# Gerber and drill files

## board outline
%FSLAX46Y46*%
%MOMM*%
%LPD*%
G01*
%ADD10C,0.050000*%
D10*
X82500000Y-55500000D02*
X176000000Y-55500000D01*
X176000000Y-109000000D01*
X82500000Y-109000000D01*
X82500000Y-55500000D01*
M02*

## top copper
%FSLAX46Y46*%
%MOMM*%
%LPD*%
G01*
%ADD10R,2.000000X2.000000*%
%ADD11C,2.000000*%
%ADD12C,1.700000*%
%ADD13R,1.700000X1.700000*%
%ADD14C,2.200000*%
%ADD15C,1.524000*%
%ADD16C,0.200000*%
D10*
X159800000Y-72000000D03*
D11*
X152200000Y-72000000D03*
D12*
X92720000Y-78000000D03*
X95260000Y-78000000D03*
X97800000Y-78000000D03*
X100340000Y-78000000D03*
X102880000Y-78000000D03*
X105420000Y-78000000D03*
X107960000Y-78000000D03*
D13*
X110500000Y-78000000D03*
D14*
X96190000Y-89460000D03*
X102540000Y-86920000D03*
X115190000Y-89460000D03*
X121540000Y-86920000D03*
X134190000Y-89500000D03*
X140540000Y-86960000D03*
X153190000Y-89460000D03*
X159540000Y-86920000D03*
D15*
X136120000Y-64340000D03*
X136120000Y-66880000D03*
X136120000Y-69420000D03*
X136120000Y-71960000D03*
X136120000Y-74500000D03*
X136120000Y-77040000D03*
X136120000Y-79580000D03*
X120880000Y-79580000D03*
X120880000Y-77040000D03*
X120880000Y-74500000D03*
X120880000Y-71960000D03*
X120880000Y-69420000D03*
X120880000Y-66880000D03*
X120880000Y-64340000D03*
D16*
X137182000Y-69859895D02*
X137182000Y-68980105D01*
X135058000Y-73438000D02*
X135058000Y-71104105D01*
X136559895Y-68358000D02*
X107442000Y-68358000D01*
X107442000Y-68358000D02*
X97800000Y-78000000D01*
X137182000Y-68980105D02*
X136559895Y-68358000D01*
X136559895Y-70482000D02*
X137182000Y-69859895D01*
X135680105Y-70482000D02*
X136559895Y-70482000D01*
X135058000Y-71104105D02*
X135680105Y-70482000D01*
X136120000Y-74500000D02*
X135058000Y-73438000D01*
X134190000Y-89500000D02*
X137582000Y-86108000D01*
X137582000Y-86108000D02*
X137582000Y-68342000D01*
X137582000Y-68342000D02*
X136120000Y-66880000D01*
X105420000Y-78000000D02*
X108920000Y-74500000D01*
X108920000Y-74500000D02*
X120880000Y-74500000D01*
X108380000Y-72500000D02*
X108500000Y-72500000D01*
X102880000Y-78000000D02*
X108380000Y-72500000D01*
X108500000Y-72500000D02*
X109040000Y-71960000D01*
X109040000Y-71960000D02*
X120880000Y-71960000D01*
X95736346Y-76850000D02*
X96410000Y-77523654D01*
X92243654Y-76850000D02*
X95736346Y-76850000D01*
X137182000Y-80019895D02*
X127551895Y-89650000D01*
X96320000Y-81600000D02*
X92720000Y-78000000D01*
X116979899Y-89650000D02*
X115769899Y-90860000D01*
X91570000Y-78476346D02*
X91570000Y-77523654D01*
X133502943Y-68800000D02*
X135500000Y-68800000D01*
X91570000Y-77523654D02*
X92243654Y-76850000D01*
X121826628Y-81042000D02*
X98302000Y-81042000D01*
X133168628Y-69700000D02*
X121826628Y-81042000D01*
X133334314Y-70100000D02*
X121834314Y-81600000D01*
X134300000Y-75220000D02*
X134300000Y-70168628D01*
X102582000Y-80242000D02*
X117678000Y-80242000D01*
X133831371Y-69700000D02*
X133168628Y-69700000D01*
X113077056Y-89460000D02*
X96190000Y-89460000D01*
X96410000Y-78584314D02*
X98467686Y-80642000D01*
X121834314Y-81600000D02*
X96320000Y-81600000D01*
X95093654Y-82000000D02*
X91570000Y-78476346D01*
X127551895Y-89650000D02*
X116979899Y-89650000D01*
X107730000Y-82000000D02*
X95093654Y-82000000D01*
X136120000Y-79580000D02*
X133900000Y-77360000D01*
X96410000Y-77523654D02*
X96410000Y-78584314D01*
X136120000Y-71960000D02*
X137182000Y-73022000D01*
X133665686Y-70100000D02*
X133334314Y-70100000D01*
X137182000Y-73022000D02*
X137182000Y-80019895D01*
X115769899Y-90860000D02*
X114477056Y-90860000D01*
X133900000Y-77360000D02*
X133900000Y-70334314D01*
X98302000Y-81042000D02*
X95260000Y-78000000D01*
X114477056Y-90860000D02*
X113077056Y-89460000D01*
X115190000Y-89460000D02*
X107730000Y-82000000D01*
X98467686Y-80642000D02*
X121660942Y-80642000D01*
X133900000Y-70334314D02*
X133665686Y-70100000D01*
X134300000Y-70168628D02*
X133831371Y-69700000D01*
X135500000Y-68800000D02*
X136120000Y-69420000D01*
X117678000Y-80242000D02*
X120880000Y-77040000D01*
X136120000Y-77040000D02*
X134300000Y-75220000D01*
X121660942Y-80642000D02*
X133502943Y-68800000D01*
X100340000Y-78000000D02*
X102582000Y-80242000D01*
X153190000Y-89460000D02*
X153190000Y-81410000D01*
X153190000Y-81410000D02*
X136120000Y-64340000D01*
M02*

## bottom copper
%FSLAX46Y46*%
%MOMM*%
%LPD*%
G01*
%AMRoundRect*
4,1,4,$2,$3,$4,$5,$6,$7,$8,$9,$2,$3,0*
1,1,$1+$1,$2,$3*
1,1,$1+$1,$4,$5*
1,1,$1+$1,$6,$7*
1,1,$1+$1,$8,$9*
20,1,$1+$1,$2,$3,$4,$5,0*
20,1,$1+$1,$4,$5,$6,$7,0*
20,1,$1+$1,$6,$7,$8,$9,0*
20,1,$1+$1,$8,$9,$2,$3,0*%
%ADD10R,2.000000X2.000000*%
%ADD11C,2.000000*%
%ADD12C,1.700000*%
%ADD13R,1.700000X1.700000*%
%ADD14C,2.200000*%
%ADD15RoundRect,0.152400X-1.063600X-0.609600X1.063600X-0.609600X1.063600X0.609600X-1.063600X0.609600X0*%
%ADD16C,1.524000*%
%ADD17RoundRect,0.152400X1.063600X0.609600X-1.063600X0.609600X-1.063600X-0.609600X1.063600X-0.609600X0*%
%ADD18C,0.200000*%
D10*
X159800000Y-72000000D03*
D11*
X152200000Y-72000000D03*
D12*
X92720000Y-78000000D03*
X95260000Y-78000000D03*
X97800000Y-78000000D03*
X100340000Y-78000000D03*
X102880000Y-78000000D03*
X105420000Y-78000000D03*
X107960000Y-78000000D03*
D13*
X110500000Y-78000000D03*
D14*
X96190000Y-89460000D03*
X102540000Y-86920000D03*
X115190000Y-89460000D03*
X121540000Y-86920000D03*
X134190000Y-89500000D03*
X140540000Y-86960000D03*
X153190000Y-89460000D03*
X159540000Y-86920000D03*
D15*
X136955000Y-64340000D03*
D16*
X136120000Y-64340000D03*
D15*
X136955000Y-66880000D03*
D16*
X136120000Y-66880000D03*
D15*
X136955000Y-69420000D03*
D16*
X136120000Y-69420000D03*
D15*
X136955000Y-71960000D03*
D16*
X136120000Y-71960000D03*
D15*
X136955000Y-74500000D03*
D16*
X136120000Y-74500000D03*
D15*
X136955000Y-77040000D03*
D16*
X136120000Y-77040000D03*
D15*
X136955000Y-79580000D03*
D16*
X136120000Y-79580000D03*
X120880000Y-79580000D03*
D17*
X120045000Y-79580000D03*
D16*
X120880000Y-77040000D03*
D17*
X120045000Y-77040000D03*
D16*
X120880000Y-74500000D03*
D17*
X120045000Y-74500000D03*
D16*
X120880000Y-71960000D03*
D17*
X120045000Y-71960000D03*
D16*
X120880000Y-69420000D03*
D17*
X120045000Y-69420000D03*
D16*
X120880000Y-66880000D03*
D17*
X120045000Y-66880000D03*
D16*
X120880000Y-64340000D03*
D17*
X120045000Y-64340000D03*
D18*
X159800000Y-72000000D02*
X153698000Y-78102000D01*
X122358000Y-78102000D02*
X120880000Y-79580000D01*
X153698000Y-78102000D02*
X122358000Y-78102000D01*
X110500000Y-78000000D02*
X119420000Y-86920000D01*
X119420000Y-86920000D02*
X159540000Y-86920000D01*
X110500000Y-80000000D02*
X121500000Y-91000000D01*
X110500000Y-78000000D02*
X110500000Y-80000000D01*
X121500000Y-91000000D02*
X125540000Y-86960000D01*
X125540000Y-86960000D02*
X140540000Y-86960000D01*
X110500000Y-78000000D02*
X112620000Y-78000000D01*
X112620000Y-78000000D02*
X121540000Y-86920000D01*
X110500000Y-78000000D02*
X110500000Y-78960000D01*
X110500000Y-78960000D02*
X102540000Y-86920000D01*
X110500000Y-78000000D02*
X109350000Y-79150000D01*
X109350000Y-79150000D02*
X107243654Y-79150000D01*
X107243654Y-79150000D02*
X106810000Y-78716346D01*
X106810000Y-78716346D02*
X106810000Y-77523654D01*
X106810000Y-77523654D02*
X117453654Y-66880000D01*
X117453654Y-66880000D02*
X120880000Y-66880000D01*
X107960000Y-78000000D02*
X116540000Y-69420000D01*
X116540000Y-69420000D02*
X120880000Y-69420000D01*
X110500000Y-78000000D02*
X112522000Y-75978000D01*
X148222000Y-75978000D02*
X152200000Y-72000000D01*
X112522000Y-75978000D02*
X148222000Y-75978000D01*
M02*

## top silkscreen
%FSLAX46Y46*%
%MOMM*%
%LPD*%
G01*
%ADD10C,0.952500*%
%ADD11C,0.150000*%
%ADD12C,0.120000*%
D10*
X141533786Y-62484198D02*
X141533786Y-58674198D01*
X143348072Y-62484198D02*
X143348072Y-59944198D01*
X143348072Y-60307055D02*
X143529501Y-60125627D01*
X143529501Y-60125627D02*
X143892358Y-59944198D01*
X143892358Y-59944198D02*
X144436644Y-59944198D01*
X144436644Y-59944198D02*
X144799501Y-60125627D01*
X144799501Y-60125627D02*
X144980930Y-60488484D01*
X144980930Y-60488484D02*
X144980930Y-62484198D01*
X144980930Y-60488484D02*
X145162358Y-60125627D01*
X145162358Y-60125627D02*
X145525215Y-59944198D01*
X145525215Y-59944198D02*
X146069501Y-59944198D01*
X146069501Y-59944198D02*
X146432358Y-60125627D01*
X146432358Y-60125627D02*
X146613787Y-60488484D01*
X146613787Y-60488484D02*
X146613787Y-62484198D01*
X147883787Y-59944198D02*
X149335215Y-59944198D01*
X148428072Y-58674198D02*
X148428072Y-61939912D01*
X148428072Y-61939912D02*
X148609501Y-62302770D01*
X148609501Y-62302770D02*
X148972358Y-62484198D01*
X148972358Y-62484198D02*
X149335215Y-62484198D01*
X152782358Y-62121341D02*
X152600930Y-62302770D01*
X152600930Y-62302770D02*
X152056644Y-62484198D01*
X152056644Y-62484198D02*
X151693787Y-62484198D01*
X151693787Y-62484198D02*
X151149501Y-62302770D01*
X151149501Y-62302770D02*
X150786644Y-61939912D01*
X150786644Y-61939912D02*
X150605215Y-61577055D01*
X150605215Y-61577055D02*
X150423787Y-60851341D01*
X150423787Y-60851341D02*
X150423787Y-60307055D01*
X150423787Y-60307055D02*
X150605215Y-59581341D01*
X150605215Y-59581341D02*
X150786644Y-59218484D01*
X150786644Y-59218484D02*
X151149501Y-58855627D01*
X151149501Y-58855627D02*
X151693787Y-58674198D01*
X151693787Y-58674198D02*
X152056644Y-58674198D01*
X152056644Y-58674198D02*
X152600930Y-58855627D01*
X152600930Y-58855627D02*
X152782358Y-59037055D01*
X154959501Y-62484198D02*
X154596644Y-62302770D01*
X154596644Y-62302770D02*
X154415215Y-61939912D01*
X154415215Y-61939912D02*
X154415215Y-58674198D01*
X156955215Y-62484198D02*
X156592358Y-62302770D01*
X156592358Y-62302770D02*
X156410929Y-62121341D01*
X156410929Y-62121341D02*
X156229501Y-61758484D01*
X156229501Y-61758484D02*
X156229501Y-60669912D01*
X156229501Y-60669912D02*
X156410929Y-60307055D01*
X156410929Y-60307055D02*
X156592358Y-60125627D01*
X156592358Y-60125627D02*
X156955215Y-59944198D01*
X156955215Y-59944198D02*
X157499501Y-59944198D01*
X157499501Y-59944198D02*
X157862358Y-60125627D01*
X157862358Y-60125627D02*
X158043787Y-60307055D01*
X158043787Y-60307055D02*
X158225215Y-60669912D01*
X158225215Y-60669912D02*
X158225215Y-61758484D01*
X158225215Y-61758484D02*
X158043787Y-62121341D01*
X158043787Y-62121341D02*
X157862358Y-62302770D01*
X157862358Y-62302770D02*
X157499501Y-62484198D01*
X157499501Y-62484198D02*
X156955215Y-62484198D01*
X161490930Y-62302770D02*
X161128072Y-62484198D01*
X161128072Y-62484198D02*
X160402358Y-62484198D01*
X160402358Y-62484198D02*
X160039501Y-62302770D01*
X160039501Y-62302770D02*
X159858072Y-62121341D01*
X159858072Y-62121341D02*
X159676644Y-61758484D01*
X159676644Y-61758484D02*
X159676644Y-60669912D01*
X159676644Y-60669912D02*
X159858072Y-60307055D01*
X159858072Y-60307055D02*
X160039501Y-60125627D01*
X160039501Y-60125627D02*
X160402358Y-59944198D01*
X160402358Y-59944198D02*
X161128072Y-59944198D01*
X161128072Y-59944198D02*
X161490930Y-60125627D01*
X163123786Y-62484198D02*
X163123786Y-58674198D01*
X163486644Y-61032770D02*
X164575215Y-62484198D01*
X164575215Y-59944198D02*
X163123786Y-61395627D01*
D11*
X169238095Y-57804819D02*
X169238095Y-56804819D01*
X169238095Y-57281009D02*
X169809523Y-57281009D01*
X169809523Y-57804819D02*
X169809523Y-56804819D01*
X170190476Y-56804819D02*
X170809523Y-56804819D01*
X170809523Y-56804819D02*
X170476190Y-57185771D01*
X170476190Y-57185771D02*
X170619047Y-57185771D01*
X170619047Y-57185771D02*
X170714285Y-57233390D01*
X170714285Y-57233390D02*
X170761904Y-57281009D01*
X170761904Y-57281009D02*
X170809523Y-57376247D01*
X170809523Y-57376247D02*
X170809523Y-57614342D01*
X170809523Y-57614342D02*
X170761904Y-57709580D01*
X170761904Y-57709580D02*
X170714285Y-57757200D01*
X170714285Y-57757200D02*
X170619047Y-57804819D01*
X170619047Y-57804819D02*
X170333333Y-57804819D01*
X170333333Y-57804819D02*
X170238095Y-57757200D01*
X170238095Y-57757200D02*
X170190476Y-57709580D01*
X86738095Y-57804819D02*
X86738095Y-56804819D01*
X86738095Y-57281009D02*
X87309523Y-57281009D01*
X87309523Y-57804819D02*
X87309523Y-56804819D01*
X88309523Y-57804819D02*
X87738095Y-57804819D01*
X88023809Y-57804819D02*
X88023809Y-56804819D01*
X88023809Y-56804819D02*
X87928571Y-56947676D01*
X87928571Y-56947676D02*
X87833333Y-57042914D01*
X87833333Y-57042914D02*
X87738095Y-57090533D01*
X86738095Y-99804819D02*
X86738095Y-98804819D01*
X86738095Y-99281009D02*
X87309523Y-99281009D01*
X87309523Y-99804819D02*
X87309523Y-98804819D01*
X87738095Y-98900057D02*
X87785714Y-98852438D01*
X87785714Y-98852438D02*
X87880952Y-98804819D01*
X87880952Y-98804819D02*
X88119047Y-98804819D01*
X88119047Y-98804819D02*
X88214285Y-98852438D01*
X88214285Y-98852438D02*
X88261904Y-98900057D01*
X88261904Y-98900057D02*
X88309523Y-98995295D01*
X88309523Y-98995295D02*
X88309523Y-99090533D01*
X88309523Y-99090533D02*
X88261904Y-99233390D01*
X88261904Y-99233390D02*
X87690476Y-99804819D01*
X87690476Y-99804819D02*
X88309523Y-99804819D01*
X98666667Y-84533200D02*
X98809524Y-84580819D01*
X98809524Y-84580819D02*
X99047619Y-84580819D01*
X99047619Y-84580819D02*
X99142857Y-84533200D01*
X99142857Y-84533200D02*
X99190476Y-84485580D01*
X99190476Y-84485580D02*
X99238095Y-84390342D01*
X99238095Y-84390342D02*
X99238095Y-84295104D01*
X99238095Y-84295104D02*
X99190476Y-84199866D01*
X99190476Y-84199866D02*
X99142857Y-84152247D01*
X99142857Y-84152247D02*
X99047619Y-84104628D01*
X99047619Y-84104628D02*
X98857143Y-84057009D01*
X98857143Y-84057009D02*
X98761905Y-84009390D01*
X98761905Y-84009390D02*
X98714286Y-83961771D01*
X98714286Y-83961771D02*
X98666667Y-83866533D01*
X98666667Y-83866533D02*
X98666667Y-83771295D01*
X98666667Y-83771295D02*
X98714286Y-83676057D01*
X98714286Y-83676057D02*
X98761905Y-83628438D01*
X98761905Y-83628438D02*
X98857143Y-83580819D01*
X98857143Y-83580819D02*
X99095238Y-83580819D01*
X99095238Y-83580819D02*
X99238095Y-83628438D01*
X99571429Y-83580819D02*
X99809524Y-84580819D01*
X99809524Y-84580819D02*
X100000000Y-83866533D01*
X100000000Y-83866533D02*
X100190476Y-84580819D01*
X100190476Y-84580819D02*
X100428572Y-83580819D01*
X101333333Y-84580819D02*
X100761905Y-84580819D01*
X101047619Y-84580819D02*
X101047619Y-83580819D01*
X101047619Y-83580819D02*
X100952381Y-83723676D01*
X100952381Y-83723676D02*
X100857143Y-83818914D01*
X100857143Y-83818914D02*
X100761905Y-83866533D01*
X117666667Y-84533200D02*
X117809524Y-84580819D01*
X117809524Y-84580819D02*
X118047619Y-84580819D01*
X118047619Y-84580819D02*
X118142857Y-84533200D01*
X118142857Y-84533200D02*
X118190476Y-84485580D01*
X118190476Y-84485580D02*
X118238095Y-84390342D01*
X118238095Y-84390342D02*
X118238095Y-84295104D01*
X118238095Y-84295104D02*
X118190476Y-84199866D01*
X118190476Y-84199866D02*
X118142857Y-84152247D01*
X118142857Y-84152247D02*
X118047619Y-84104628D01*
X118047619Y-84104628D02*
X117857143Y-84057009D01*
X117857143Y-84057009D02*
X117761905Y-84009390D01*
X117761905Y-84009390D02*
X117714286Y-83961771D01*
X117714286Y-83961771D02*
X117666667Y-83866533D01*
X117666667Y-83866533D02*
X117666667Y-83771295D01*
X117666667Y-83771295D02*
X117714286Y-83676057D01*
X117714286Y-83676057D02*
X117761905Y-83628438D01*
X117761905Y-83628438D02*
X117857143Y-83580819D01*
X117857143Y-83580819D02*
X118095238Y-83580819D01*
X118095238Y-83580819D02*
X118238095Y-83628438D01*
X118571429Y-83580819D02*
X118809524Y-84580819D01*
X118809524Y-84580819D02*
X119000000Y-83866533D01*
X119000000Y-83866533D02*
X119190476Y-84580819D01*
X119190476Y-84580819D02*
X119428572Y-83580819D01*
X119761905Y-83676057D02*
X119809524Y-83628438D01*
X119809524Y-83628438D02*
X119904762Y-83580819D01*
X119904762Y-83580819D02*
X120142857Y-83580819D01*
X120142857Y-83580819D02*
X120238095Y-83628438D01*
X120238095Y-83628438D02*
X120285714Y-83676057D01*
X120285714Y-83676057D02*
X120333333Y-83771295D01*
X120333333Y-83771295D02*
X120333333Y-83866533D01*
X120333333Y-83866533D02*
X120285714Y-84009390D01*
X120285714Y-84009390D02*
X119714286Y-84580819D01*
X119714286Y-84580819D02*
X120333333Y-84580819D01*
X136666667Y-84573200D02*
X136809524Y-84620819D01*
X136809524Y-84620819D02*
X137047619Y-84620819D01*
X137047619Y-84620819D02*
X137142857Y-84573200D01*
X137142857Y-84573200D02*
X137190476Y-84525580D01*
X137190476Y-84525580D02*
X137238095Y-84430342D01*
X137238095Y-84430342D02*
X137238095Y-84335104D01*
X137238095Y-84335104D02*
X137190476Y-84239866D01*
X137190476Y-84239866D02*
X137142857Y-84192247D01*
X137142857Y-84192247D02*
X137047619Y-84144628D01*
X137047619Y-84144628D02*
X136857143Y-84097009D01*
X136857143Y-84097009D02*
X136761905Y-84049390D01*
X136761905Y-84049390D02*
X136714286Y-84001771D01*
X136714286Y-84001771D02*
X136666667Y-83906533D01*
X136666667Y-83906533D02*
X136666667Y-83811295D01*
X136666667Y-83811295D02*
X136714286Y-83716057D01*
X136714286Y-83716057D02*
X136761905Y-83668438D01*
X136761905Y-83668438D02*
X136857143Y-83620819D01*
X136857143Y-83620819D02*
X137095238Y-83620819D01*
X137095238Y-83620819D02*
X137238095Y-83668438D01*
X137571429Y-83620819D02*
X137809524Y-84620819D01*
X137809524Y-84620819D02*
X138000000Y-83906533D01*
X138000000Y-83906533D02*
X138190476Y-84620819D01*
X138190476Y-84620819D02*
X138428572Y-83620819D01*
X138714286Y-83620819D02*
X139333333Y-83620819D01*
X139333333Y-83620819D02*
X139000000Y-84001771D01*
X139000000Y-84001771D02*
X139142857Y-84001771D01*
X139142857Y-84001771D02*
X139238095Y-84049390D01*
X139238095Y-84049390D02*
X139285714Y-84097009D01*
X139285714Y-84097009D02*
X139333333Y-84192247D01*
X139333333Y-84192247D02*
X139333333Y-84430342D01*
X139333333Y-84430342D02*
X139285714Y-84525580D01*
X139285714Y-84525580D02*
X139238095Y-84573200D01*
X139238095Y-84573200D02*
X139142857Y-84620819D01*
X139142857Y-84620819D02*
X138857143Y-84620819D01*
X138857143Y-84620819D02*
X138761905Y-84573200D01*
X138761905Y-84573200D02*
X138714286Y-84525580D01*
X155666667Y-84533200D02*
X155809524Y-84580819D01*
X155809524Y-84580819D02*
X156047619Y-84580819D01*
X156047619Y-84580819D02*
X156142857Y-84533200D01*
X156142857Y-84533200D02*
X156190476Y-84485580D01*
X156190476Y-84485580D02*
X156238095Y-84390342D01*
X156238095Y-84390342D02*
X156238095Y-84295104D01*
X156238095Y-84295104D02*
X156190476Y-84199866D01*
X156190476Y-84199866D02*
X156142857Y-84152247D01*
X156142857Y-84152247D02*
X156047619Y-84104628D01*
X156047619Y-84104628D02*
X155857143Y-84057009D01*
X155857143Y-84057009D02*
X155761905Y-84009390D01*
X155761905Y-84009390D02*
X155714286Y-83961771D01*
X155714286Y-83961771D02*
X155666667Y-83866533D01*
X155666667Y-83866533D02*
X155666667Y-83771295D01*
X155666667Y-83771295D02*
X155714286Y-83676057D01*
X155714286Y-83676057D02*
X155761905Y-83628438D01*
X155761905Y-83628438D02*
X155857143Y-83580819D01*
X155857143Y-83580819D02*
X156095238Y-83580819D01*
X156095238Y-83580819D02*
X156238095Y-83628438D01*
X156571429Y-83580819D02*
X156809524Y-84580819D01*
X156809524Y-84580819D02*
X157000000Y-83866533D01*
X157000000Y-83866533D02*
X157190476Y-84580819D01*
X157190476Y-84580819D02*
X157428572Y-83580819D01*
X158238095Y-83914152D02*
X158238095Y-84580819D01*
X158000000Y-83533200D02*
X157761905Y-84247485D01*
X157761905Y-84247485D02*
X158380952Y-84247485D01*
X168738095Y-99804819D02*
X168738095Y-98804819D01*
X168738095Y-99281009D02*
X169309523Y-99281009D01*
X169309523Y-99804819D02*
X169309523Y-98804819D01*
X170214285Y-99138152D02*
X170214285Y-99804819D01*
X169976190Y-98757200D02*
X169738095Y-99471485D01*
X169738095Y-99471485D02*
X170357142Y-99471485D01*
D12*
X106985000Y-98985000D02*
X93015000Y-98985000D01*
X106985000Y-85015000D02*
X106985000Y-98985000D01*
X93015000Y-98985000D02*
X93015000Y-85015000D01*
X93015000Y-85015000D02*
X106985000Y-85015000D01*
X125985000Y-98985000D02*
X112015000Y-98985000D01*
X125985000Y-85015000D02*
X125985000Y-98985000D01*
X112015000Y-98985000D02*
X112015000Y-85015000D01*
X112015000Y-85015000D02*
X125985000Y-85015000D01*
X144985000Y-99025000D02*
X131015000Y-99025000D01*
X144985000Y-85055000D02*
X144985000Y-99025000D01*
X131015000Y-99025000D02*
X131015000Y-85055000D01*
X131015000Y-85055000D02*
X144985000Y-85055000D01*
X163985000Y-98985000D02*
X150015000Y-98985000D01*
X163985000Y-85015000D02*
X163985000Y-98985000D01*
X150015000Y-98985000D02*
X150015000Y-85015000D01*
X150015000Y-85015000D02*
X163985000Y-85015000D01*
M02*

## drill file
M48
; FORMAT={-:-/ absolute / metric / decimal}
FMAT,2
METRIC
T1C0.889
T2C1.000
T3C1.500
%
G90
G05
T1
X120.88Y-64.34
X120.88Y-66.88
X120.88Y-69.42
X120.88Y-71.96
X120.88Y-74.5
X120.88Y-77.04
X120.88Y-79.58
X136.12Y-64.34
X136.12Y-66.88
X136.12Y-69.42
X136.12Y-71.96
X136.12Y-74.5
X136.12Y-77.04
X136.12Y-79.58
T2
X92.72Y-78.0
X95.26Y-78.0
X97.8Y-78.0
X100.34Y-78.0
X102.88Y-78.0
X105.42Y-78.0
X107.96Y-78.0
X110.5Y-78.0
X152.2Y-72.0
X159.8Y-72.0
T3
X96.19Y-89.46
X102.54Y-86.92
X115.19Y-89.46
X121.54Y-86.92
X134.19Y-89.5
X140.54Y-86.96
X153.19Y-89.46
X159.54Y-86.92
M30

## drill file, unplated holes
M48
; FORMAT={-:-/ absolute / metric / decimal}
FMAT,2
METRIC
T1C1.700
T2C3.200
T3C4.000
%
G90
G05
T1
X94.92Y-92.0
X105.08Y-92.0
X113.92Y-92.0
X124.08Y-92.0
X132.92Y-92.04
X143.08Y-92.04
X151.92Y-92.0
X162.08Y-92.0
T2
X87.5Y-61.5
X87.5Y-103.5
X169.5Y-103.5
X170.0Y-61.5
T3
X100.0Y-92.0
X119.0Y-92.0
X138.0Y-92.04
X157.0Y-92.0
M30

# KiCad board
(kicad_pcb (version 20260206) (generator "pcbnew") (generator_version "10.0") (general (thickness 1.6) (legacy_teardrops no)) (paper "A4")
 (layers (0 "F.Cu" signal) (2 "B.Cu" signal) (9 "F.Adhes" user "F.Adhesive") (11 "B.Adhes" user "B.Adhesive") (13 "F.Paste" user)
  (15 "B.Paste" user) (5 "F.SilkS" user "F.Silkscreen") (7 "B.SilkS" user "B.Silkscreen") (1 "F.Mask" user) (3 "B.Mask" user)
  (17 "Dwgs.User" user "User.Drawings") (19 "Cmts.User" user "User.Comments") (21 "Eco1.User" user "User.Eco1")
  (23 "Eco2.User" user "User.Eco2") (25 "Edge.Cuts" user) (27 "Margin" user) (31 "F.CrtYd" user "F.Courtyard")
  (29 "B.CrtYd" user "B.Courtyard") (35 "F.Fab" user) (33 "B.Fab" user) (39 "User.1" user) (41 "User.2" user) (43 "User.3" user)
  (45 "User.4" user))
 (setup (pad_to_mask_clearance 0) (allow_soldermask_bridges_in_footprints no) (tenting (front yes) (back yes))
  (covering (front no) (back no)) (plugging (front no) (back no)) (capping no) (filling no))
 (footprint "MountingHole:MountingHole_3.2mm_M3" (layer "F.Cu") (at 169.5 103.5)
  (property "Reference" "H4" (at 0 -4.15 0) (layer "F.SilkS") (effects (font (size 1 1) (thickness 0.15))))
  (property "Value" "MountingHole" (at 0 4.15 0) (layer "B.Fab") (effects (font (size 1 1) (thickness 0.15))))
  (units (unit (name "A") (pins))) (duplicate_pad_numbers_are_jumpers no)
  (pad "" np_thru_hole circle (at 0 0) (size 3.2 3.2) (drill 3.2) (layers "*.Cu" "*.Mask")))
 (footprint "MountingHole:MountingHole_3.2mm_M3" (layer "F.Cu") (at 87.5 61.5)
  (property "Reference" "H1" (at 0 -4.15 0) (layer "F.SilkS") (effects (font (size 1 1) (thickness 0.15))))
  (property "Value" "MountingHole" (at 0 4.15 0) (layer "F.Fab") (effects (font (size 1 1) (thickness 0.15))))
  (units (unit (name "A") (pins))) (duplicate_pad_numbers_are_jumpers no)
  (pad "" np_thru_hole circle (at 0 0) (size 3.2 3.2) (drill 3.2) (layers "*.Cu" "*.Mask")))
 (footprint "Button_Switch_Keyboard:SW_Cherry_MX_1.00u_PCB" (layer "F.Cu") (at 159.54 86.92)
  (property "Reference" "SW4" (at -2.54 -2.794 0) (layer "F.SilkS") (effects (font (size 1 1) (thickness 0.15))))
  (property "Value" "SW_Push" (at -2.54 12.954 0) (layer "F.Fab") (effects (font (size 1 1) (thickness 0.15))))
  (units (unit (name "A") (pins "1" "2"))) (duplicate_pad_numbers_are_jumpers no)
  (fp_line (start -9.525 -1.905) (end 4.445 -1.905) (stroke (width 0.12) (type solid)) (layer "F.SilkS"))
  (fp_line (start -9.525 12.065) (end -9.525 -1.905) (stroke (width 0.12) (type solid)) (layer "F.SilkS"))
  (fp_line (start 4.445 -1.905) (end 4.445 12.065) (stroke (width 0.12) (type solid)) (layer "F.SilkS"))
  (fp_line (start 4.445 12.065) (end -9.525 12.065) (stroke (width 0.12) (type solid)) (layer "F.SilkS"))
  (pad "" np_thru_hole circle (at -7.62 5.08) (size 1.7 1.7) (drill 1.7) (layers "*.Cu" "*.Mask"))
  (pad "" np_thru_hole circle (at -2.54 5.08) (size 4 4) (drill 4) (layers "*.Cu" "*.Mask"))
  (pad "" np_thru_hole circle (at 2.54 5.08) (size 1.7 1.7) (drill 1.7) (layers "*.Cu" "*.Mask"))
  (pad "1" thru_hole circle (at 0 0) (size 2.2 2.2) (drill 1.5) (layers "*.Cu" "*.Mask") (remove_unused_layers no) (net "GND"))
  (pad "2" thru_hole circle (at -6.35 2.54) (size 2.2 2.2) (drill 1.5) (layers "*.Cu" "*.Mask") (remove_unused_layers no)
   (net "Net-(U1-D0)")))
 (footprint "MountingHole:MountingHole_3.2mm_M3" (layer "F.Cu") (at 170 61.5)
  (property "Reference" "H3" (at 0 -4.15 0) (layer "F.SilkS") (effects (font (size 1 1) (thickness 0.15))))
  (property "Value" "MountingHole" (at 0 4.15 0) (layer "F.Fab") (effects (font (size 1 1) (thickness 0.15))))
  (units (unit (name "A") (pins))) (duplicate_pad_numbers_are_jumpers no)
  (pad "" np_thru_hole circle (at 0 0) (size 3.2 3.2) (drill 3.2) (layers "*.Cu" "*.Mask")))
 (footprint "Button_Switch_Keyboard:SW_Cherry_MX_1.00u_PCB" (layer "F.Cu") (at 140.54 86.96)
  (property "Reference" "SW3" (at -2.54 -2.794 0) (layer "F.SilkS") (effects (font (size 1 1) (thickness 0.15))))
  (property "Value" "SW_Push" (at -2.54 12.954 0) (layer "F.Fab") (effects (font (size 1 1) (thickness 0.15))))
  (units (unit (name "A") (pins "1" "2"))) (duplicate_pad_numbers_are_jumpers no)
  (fp_line (start -9.525 -1.905) (end 4.445 -1.905) (stroke (width 0.12) (type solid)) (layer "F.SilkS"))
  (fp_line (start -9.525 12.065) (end -9.525 -1.905) (stroke (width 0.12) (type solid)) (layer "F.SilkS"))
  (fp_line (start 4.445 -1.905) (end 4.445 12.065) (stroke (width 0.12) (type solid)) (layer "F.SilkS"))
  (fp_line (start 4.445 12.065) (end -9.525 12.065) (stroke (width 0.12) (type solid)) (layer "F.SilkS"))
  (pad "" np_thru_hole circle (at -7.62 5.08) (size 1.7 1.7) (drill 1.7) (layers "*.Cu" "*.Mask"))
  (pad "" np_thru_hole circle (at -2.54 5.08) (size 4 4) (drill 4) (layers "*.Cu" "*.Mask"))
  (pad "" np_thru_hole circle (at 2.54 5.08) (size 1.7 1.7) (drill 1.7) (layers "*.Cu" "*.Mask"))
  (pad "1" thru_hole circle (at 0 0) (size 2.2 2.2) (drill 1.5) (layers "*.Cu" "*.Mask") (remove_unused_layers no) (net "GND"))
  (pad "2" thru_hole circle (at -6.35 2.54) (size 2.2 2.2) (drill 1.5) (layers "*.Cu" "*.Mask") (remove_unused_layers no)
   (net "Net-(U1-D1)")))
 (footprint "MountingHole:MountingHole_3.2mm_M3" (layer "F.Cu") (at 87.5 103.5)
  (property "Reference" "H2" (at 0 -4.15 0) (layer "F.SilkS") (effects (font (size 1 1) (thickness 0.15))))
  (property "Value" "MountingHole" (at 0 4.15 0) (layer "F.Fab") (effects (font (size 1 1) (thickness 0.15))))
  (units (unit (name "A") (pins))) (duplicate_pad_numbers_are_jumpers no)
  (pad "" np_thru_hole circle (at 0 0) (size 3.2 3.2) (drill 3.2) (layers "*.Cu" "*.Mask")))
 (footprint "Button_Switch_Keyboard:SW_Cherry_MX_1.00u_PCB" (layer "F.Cu") (at 121.54 86.92)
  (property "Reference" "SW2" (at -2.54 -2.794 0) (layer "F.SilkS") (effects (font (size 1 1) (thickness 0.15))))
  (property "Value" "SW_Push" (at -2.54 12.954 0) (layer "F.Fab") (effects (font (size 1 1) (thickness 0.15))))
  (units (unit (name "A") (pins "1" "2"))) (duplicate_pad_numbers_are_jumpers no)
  (fp_line (start -9.525 -1.905) (end 4.445 -1.905) (stroke (width 0.12) (type solid)) (layer "F.SilkS"))
  (fp_line (start -9.525 12.065) (end -9.525 -1.905) (stroke (width 0.12) (type solid)) (layer "F.SilkS"))
  (fp_line (start 4.445 -1.905) (end 4.445 12.065) (stroke (width 0.12) (type solid)) (layer "F.SilkS"))
  (fp_line (start 4.445 12.065) (end -9.525 12.065) (stroke (width 0.12) (type solid)) (layer "F.SilkS"))
  (pad "" np_thru_hole circle (at -7.62 5.08) (size 1.7 1.7) (drill 1.7) (layers "*.Cu" "*.Mask"))
  (pad "" np_thru_hole circle (at -2.54 5.08) (size 4 4) (drill 4) (layers "*.Cu" "*.Mask"))
  (pad "" np_thru_hole circle (at 2.54 5.08) (size 1.7 1.7) (drill 1.7) (layers "*.Cu" "*.Mask"))
  (pad "1" thru_hole circle (at 0 0) (size 2.2 2.2) (drill 1.5) (layers "*.Cu" "*.Mask") (remove_unused_layers no) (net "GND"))
  (pad "2" thru_hole circle (at -6.35 2.54) (size 2.2 2.2) (drill 1.5) (layers "*.Cu" "*.Mask") (remove_unused_layers no)
   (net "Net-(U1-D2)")))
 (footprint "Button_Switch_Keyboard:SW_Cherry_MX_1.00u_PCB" (layer "F.Cu") (at 102.54 86.92)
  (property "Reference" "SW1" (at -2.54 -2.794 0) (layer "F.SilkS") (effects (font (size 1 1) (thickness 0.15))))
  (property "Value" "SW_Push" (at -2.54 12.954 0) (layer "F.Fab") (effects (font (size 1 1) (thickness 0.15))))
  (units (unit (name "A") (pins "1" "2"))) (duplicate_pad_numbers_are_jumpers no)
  (fp_line (start -9.525 -1.905) (end 4.445 -1.905) (stroke (width 0.12) (type solid)) (layer "F.SilkS"))
  (fp_line (start -9.525 12.065) (end -9.525 -1.905) (stroke (width 0.12) (type solid)) (layer "F.SilkS"))
  (fp_line (start 4.445 -1.905) (end 4.445 12.065) (stroke (width 0.12) (type solid)) (layer "F.SilkS"))
  (fp_line (start 4.445 12.065) (end -9.525 12.065) (stroke (width 0.12) (type solid)) (layer "F.SilkS"))
  (pad "" np_thru_hole circle (at -7.62 5.08) (size 1.7 1.7) (drill 1.7) (layers "*.Cu" "*.Mask"))
  (pad "" np_thru_hole circle (at -2.54 5.08) (size 4 4) (drill 4) (layers "*.Cu" "*.Mask"))
  (pad "" np_thru_hole circle (at 2.54 5.08) (size 1.7 1.7) (drill 1.7) (layers "*.Cu" "*.Mask"))
  (pad "1" thru_hole circle (at 0 0) (size 2.2 2.2) (drill 1.5) (layers "*.Cu" "*.Mask") (remove_unused_layers no) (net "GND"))
  (pad "2" thru_hole circle (at -6.35 2.54) (size 2.2 2.2) (drill 1.5) (layers "*.Cu" "*.Mask") (remove_unused_layers no)
   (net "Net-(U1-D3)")))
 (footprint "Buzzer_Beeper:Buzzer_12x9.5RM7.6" (layer "B.Cu") (at 159.8 72 180)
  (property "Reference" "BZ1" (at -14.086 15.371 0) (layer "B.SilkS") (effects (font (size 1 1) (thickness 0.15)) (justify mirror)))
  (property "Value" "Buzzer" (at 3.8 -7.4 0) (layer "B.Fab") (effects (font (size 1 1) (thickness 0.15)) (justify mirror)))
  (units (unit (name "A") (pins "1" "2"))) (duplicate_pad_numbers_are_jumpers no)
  (pad "1" thru_hole rect (at 0 0 180) (size 2 2) (drill 1) (layers "*.Cu" "*.Mask") (remove_unused_layers no) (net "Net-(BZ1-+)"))
  (pad "2" thru_hole circle (at 7.6 0 180) (size 2 2) (drill 1) (layers "*.Cu" "*.Mask") (remove_unused_layers no) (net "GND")))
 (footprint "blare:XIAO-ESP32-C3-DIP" (layer "B.Cu") (at 128.5 71.96 90)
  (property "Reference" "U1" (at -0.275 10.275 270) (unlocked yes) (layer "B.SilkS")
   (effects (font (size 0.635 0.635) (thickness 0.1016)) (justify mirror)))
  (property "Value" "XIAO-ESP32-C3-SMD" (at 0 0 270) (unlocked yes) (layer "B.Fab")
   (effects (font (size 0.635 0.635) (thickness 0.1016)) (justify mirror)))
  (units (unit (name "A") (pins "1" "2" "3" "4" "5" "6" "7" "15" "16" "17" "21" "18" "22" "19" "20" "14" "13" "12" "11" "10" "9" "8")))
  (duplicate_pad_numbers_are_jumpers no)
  (pad "1" thru_hole circle (at 7.62 7.62) (size 1.524 1.524) (drill 0.889) (layers "*.Cu" "*.Mask") (remove_unused_layers no)
   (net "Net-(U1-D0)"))
  (pad "1" smd roundrect (at 7.62 8.455) (size 2.432 1.524) (layers "B.Cu" "B.Mask") (roundrect_rratio 0.1) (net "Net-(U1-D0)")
   (thermal_bridge_angle 45))
  (pad "2" thru_hole circle (at 5.08 7.62) (size 1.524 1.524) (drill 0.889) (layers "*.Cu" "*.Mask") (remove_unused_layers no)
   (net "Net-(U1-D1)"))
  (pad "2" smd roundrect (at 5.08 8.455) (size 2.432 1.524) (layers "B.Cu" "B.Mask") (roundrect_rratio 0.1) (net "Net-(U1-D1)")
   (thermal_bridge_angle 45))
  (pad "3" thru_hole circle (at 2.54 7.62) (size 1.524 1.524) (drill 0.889) (layers "*.Cu" "*.Mask") (remove_unused_layers no)
   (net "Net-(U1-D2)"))
  (pad "3" smd roundrect (at 2.54 8.455) (size 2.432 1.524) (layers "B.Cu" "B.Mask") (roundrect_rratio 0.1) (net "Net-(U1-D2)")
   (thermal_bridge_angle 45))
  (pad "4" thru_hole circle (at 0 7.62) (size 1.524 1.524) (drill 0.889) (layers "*.Cu" "*.Mask") (remove_unused_layers no)
   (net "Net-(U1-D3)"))
  (pad "4" smd roundrect (at 0 8.455) (size 2.432 1.524) (layers "B.Cu" "B.Mask") (roundrect_rratio 0.1) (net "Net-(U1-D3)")
   (thermal_bridge_angle 45))
  (pad "5" thru_hole circle (at -2.54 7.62) (size 1.524 1.524) (drill 0.889) (layers "*.Cu" "*.Mask") (remove_unused_layers no) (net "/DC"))
  (pad "5" smd roundrect (at -2.54 8.455) (size 2.432 1.524) (layers "B.Cu" "B.Mask") (roundrect_rratio 0.1) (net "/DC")
   (thermal_bridge_angle 45))
  (pad "6" thru_hole circle (at -5.08 7.62) (size 1.524 1.524) (drill 0.889) (layers "*.Cu" "*.Mask") (remove_unused_layers no) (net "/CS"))
  (pad "6" smd roundrect (at -5.08 8.455) (size 2.432 1.524) (layers "B.Cu" "B.Mask") (roundrect_rratio 0.1) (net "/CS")
   (thermal_bridge_angle 45))
  (pad "7" thru_hole circle (at -7.62 7.62) (size 1.524 1.524) (drill 0.889) (layers "*.Cu" "*.Mask") (remove_unused_layers no) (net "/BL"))
  (pad "7" smd roundrect (at -7.62 8.455) (size 2.432 1.524) (layers "B.Cu" "B.Mask") (roundrect_rratio 0.1) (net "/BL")
   (thermal_bridge_angle 45))
  (pad "8" smd roundrect (at -7.62 -8.455 180) (size 2.432 1.524) (layers "B.Cu" "B.Mask") (roundrect_rratio 0.1) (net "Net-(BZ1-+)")
   (thermal_bridge_angle 45))
  (pad "8" thru_hole circle (at -7.62 -7.62 180) (size 1.524 1.524) (drill 0.889) (layers "*.Cu" "*.Mask") (remove_unused_layers no)
   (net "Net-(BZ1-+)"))
  (pad "9" smd roundrect (at -5.08 -8.455 180) (size 2.432 1.524) (layers "B.Cu" "B.Mask") (roundrect_rratio 0.1) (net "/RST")
   (thermal_bridge_angle 45))
  (pad "9" thru_hole circle (at -5.08 -7.62 180) (size 1.524 1.524) (drill 0.889) (layers "*.Cu" "*.Mask") (remove_unused_layers no)
   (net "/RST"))
  (pad "10" smd roundrect (at -2.54 -8.455 180) (size 2.432 1.524) (layers "B.Cu" "B.Mask") (roundrect_rratio 0.1) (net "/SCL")
   (thermal_bridge_angle 45))
  (pad "10" thru_hole circle (at -2.54 -7.62 180) (size 1.524 1.524) (drill 0.889) (layers "*.Cu" "*.Mask") (remove_unused_layers no)
   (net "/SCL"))
  (pad "11" smd roundrect (at 0 -8.455 180) (size 2.432 1.524) (layers "B.Cu" "B.Mask") (roundrect_rratio 0.1) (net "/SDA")
   (thermal_bridge_angle 45))
  (pad "11" thru_hole circle (at 0 -7.62 180) (size 1.524 1.524) (drill 0.889) (layers "*.Cu" "*.Mask") (remove_unused_layers no)
   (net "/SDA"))
  (pad "12" smd roundrect (at 2.54 -8.455 180) (size 2.432 1.524) (layers "B.Cu" "B.Mask") (roundrect_rratio 0.1) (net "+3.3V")
   (thermal_bridge_angle 45))
  (pad "12" thru_hole circle (at 2.54 -7.62 180) (size 1.524 1.524) (drill 0.889) (layers "*.Cu" "*.Mask") (remove_unused_layers no)
   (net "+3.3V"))
  (pad "13" smd roundrect (at 5.08 -8.455 180) (size 2.432 1.524) (layers "B.Cu" "B.Mask") (roundrect_rratio 0.1) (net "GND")
   (thermal_bridge_angle 45))
  (pad "13" thru_hole circle (at 5.08 -7.62 180) (size 1.524 1.524) (drill 0.889) (layers "*.Cu" "*.Mask") (remove_unused_layers no)
   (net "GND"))
  (pad "14" smd roundrect (at 7.62 -8.455 180) (size 2.432 1.524) (layers "B.Cu" "B.Mask") (roundrect_rratio 0.1)
   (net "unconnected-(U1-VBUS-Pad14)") (thermal_bridge_angle 45))
  (pad "14" thru_hole circle (at 7.62 -7.62 180) (size 1.524 1.524) (drill 0.889) (layers "*.Cu" "*.Mask") (remove_unused_layers no)
   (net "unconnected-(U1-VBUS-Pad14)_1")))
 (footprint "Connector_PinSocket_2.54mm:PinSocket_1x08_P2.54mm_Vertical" (layer "B.Cu") (at 110.5 78 90)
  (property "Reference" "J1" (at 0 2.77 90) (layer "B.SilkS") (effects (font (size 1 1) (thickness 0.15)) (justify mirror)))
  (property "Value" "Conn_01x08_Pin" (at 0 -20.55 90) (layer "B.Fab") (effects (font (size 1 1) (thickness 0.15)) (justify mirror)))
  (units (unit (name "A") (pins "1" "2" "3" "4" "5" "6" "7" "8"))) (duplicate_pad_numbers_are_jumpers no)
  (pad "1" thru_hole rect (at 0 0 90) (size 1.7 1.7) (drill 1) (layers "*.Cu" "*.Mask") (remove_unused_layers no) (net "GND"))
  (pad "2" thru_hole circle (at 0 -2.54 90) (size 1.7 1.7) (drill 1) (layers "*.Cu" "*.Mask") (remove_unused_layers no) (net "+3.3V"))
  (pad "3" thru_hole circle (at 0 -5.08 90) (size 1.7 1.7) (drill 1) (layers "*.Cu" "*.Mask") (remove_unused_layers no) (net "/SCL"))
  (pad "4" thru_hole circle (at 0 -7.62 90) (size 1.7 1.7) (drill 1) (layers "*.Cu" "*.Mask") (remove_unused_layers no) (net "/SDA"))
  (pad "5" thru_hole circle (at 0 -10.16 90) (size 1.7 1.7) (drill 1) (layers "*.Cu" "*.Mask") (remove_unused_layers no) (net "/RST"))
  (pad "6" thru_hole circle (at 0 -12.7 90) (size 1.7 1.7) (drill 1) (layers "*.Cu" "*.Mask") (remove_unused_layers no) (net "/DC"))
  (pad "7" thru_hole circle (at 0 -15.24 90) (size 1.7 1.7) (drill 1) (layers "*.Cu" "*.Mask") (remove_unused_layers no) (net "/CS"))
  (pad "8" thru_hole circle (at 0 -17.78 90) (size 1.7 1.7) (drill 1) (layers "*.Cu" "*.Mask") (remove_unused_layers no) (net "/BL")))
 (gr_rect (start 82.5 55.5) (end 176 109) (stroke (width 0.05) (type default)) (fill no) (layer "Edge.Cuts"))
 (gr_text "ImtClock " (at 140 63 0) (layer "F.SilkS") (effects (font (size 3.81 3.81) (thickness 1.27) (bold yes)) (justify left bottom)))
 (segment (start 112.522 75.978) (end 148.222 75.978) (width 0.2) (layer "B.Cu") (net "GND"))
 (segment (start 110.5 78) (end 110.5 80) (width 0.2) (layer "B.Cu") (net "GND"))
 (segment (start 110.5 78) (end 112.522 75.978) (width 0.2) (layer "B.Cu") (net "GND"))
 (segment (start 110.5 78) (end 112.62 78) (width 0.2) (layer "B.Cu") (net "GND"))
 (segment (start 109.35 79.15) (end 107.243654 79.15) (width 0.2) (layer "B.Cu") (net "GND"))
 (segment (start 117.453654 66.88) (end 120.88 66.88) (width 0.2) (layer "B.Cu") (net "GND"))
 (segment (start 112.62 78) (end 121.54 86.92) (width 0.2) (layer "B.Cu") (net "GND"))
 (segment (start 107.243654 79.15) (end 106.81 78.716346) (width 0.2) (layer "B.Cu") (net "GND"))
 (segment (start 110.5 78.96) (end 102.54 86.92) (width 0.2) (layer "B.Cu") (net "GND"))
 (segment (start 110.5 80) (end 121.5 91) (width 0.2) (layer "B.Cu") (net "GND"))
 (segment (start 106.81 77.523654) (end 117.453654 66.88) (width 0.2) (layer "B.Cu") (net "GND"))
 (segment (start 148.222 75.978) (end 152.2 72) (width 0.2) (layer "B.Cu") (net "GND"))
 (segment (start 121.5 91) (end 125.54 86.96) (width 0.2) (layer "B.Cu") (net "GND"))
 (segment (start 110.5 78) (end 119.42 86.92) (width 0.2) (layer "B.Cu") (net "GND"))
 (segment (start 110.5 78) (end 110.5 78.96) (width 0.2) (layer "B.Cu") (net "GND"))
 (segment (start 125.54 86.96) (end 140.54 86.96) (width 0.2) (layer "B.Cu") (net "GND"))
 (segment (start 119.42 86.92) (end 159.54 86.92) (width 0.2) (layer "B.Cu") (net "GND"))
 (segment (start 106.81 78.716346) (end 106.81 77.523654) (width 0.2) (layer "B.Cu") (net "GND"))
 (segment (start 110.5 78) (end 109.35 79.15) (width 0.2) (layer "B.Cu") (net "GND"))
 (segment (start 122.358 78.102) (end 120.88 79.58) (width 0.2) (layer "B.Cu") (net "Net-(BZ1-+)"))
 (segment (start 159.8 72) (end 153.698 78.102) (width 0.2) (layer "B.Cu") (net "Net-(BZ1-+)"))
 (segment (start 153.698 78.102) (end 122.358 78.102) (width 0.2) (layer "B.Cu") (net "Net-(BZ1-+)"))
 (segment (start 137.182 68.980105) (end 136.559895 68.358) (width 0.2) (layer "F.Cu") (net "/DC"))
 (segment (start 135.680105 70.482) (end 136.559895 70.482) (width 0.2) (layer "F.Cu") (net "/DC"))
 (segment (start 137.182 69.859895) (end 137.182 68.980105) (width 0.2) (layer "F.Cu") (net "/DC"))
 (segment (start 136.559895 68.358) (end 107.442 68.358) (width 0.2) (layer "F.Cu") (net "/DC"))
 (segment (start 135.058 73.438) (end 135.058 71.104105) (width 0.2) (layer "F.Cu") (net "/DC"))
 (segment (start 136.12 74.5) (end 135.058 73.438) (width 0.2) (layer "F.Cu") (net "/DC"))
 (segment (start 135.058 71.104105) (end 135.680105 70.482) (width 0.2) (layer "F.Cu") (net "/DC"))
 (segment (start 136.559895 70.482) (end 137.182 69.859895) (width 0.2) (layer "F.Cu") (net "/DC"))
 (segment (start 107.442 68.358) (end 97.8 78) (width 0.2) (layer "F.Cu") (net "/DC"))
 (segment (start 133.831371 69.7) (end 133.168628 69.7) (width 0.2) (layer "F.Cu") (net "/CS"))
 (segment (start 136.12 77.04) (end 134.3 75.22) (width 0.2) (layer "F.Cu") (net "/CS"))
 (segment (start 134.3 70.168628) (end 133.831371 69.7) (width 0.2) (layer "F.Cu") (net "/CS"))
 (segment (start 134.3 75.22) (end 134.3 70.168628) (width 0.2) (layer "F.Cu") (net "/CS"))
 (segment (start 98.302 81.042) (end 95.26 78) (width 0.2) (layer "F.Cu") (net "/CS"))
 (segment (start 133.168628 69.7) (end 121.826628 81.042) (width 0.2) (layer "F.Cu") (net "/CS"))
 (segment (start 121.826628 81.042) (end 98.302 81.042) (width 0.2) (layer "F.Cu") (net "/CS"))
 (segment (start 102.582 80.242) (end 117.678 80.242) (width 0.2) (layer "F.Cu") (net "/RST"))
 (segment (start 117.678 80.242) (end 120.88 77.04) (width 0.2) (layer "F.Cu") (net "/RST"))
 (segment (start 100.34 78) (end 102.582 80.242) (width 0.2) (layer "F.Cu") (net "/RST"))
 (segment (start 133.665686 70.1) (end 133.334314 70.1) (width 0.2) (layer "F.Cu") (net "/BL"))
 (segment (start 133.9 70.334314) (end 133.665686 70.1) (width 0.2) (layer "F.Cu") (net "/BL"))
 (segment (start 133.9 77.36) (end 133.9 70.334314) (width 0.2) (layer "F.Cu") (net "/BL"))
 (segment (start 96.32 81.6) (end 92.72 78) (width 0.2) (layer "F.Cu") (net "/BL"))
 (segment (start 121.834314 81.6) (end 96.32 81.6) (width 0.2) (layer "F.Cu") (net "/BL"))
 (segment (start 136.12 79.58) (end 133.9 77.36) (width 0.2) (layer "F.Cu") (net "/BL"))
 (segment (start 133.334314 70.1) (end 121.834314 81.6) (width 0.2) (layer "F.Cu") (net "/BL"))
 (segment (start 108.92 74.5) (end 120.88 74.5) (width 0.2) (layer "F.Cu") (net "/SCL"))
 (segment (start 105.42 78) (end 108.92 74.5) (width 0.2) (layer "F.Cu") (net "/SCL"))
 (segment (start 107.96 78) (end 116.54 69.42) (width 0.2) (layer "B.Cu") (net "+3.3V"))
 (segment (start 116.54 69.42) (end 120.88 69.42) (width 0.2) (layer "B.Cu") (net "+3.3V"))
 (segment (start 109.04 71.96) (end 120.88 71.96) (width 0.2) (layer "F.Cu") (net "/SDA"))
 (segment (start 108.38 72.5) (end 108.5 72.5) (width 0.2) (layer "F.Cu") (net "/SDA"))
 (segment (start 108.5 72.5) (end 109.04 71.96) (width 0.2) (layer "F.Cu") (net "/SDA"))
 (segment (start 102.88 78) (end 108.38 72.5) (width 0.2) (layer "F.Cu") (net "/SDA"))
 (segment (start 136.12 71.96) (end 137.182 73.022) (width 0.2) (layer "F.Cu") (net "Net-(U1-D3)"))
 (segment (start 137.182 73.022) (end 137.182 80.019895) (width 0.2) (layer "F.Cu") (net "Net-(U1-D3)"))
 (segment (start 115.769899 90.86) (end 114.477056 90.86) (width 0.2) (layer "F.Cu") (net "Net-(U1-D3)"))
 (segment (start 116.979899 89.65) (end 115.769899 90.86) (width 0.2) (layer "F.Cu") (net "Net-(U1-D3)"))
 (segment (start 127.551895 89.65) (end 116.979899 89.65) (width 0.2) (layer "F.Cu") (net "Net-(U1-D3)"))
 (segment (start 113.077056 89.46) (end 96.19 89.46) (width 0.2) (layer "F.Cu") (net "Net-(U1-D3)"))
 (segment (start 114.477056 90.86) (end 113.077056 89.46) (width 0.2) (layer "F.Cu") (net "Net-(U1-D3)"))
 (segment (start 137.182 80.019895) (end 127.551895 89.65) (width 0.2) (layer "F.Cu") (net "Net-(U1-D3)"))
 (segment (start 107.73 82) (end 95.093654 82) (width 0.2) (layer "F.Cu") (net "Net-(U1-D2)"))
 (segment (start 92.243654 76.85) (end 95.736346 76.85) (width 0.2) (layer "F.Cu") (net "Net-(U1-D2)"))
 (segment (start 98.467686 80.642) (end 121.660942 80.642) (width 0.2) (layer "F.Cu") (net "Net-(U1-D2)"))
 (segment (start 95.736346 76.85) (end 96.41 77.523654) (width 0.2) (layer "F.Cu") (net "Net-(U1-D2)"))
 (segment (start 135.5 68.8) (end 136.12 69.42) (width 0.2) (layer "F.Cu") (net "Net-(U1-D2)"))
 (segment (start 95.093654 82) (end 91.57 78.476346) (width 0.2) (layer "F.Cu") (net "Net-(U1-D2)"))
 (segment (start 133.502943 68.8) (end 135.5 68.8) (width 0.2) (layer "F.Cu") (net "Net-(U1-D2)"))
 (segment (start 96.41 77.523654) (end 96.41 78.584314) (width 0.2) (layer "F.Cu") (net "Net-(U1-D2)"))
 (segment (start 115.19 89.46) (end 107.73 82) (width 0.2) (layer "F.Cu") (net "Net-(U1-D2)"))
 (segment (start 91.57 77.523654) (end 92.243654 76.85) (width 0.2) (layer "F.Cu") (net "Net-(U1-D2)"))
 (segment (start 96.41 78.584314) (end 98.467686 80.642) (width 0.2) (layer "F.Cu") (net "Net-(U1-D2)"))
 (segment (start 91.57 78.476346) (end 91.57 77.523654) (width 0.2) (layer "F.Cu") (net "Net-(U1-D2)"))
 (segment (start 121.660942 80.642) (end 133.502943 68.8) (width 0.2) (layer "F.Cu") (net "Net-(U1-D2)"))
 (segment (start 134.19 89.5) (end 137.582 86.108) (width 0.2) (layer "F.Cu") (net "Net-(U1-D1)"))
 (segment (start 137.582 68.342) (end 136.12 66.88) (width 0.2) (layer "F.Cu") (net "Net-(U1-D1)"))
 (segment (start 137.582 86.108) (end 137.582 68.342) (width 0.2) (layer "F.Cu") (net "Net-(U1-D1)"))
 (segment (start 153.19 89.46) (end 153.19 81.41) (width 0.2) (layer "F.Cu") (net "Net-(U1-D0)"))
 (segment (start 153.19 81.41) (end 136.12 64.34) (width 0.2) (layer "F.Cu") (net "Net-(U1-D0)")))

